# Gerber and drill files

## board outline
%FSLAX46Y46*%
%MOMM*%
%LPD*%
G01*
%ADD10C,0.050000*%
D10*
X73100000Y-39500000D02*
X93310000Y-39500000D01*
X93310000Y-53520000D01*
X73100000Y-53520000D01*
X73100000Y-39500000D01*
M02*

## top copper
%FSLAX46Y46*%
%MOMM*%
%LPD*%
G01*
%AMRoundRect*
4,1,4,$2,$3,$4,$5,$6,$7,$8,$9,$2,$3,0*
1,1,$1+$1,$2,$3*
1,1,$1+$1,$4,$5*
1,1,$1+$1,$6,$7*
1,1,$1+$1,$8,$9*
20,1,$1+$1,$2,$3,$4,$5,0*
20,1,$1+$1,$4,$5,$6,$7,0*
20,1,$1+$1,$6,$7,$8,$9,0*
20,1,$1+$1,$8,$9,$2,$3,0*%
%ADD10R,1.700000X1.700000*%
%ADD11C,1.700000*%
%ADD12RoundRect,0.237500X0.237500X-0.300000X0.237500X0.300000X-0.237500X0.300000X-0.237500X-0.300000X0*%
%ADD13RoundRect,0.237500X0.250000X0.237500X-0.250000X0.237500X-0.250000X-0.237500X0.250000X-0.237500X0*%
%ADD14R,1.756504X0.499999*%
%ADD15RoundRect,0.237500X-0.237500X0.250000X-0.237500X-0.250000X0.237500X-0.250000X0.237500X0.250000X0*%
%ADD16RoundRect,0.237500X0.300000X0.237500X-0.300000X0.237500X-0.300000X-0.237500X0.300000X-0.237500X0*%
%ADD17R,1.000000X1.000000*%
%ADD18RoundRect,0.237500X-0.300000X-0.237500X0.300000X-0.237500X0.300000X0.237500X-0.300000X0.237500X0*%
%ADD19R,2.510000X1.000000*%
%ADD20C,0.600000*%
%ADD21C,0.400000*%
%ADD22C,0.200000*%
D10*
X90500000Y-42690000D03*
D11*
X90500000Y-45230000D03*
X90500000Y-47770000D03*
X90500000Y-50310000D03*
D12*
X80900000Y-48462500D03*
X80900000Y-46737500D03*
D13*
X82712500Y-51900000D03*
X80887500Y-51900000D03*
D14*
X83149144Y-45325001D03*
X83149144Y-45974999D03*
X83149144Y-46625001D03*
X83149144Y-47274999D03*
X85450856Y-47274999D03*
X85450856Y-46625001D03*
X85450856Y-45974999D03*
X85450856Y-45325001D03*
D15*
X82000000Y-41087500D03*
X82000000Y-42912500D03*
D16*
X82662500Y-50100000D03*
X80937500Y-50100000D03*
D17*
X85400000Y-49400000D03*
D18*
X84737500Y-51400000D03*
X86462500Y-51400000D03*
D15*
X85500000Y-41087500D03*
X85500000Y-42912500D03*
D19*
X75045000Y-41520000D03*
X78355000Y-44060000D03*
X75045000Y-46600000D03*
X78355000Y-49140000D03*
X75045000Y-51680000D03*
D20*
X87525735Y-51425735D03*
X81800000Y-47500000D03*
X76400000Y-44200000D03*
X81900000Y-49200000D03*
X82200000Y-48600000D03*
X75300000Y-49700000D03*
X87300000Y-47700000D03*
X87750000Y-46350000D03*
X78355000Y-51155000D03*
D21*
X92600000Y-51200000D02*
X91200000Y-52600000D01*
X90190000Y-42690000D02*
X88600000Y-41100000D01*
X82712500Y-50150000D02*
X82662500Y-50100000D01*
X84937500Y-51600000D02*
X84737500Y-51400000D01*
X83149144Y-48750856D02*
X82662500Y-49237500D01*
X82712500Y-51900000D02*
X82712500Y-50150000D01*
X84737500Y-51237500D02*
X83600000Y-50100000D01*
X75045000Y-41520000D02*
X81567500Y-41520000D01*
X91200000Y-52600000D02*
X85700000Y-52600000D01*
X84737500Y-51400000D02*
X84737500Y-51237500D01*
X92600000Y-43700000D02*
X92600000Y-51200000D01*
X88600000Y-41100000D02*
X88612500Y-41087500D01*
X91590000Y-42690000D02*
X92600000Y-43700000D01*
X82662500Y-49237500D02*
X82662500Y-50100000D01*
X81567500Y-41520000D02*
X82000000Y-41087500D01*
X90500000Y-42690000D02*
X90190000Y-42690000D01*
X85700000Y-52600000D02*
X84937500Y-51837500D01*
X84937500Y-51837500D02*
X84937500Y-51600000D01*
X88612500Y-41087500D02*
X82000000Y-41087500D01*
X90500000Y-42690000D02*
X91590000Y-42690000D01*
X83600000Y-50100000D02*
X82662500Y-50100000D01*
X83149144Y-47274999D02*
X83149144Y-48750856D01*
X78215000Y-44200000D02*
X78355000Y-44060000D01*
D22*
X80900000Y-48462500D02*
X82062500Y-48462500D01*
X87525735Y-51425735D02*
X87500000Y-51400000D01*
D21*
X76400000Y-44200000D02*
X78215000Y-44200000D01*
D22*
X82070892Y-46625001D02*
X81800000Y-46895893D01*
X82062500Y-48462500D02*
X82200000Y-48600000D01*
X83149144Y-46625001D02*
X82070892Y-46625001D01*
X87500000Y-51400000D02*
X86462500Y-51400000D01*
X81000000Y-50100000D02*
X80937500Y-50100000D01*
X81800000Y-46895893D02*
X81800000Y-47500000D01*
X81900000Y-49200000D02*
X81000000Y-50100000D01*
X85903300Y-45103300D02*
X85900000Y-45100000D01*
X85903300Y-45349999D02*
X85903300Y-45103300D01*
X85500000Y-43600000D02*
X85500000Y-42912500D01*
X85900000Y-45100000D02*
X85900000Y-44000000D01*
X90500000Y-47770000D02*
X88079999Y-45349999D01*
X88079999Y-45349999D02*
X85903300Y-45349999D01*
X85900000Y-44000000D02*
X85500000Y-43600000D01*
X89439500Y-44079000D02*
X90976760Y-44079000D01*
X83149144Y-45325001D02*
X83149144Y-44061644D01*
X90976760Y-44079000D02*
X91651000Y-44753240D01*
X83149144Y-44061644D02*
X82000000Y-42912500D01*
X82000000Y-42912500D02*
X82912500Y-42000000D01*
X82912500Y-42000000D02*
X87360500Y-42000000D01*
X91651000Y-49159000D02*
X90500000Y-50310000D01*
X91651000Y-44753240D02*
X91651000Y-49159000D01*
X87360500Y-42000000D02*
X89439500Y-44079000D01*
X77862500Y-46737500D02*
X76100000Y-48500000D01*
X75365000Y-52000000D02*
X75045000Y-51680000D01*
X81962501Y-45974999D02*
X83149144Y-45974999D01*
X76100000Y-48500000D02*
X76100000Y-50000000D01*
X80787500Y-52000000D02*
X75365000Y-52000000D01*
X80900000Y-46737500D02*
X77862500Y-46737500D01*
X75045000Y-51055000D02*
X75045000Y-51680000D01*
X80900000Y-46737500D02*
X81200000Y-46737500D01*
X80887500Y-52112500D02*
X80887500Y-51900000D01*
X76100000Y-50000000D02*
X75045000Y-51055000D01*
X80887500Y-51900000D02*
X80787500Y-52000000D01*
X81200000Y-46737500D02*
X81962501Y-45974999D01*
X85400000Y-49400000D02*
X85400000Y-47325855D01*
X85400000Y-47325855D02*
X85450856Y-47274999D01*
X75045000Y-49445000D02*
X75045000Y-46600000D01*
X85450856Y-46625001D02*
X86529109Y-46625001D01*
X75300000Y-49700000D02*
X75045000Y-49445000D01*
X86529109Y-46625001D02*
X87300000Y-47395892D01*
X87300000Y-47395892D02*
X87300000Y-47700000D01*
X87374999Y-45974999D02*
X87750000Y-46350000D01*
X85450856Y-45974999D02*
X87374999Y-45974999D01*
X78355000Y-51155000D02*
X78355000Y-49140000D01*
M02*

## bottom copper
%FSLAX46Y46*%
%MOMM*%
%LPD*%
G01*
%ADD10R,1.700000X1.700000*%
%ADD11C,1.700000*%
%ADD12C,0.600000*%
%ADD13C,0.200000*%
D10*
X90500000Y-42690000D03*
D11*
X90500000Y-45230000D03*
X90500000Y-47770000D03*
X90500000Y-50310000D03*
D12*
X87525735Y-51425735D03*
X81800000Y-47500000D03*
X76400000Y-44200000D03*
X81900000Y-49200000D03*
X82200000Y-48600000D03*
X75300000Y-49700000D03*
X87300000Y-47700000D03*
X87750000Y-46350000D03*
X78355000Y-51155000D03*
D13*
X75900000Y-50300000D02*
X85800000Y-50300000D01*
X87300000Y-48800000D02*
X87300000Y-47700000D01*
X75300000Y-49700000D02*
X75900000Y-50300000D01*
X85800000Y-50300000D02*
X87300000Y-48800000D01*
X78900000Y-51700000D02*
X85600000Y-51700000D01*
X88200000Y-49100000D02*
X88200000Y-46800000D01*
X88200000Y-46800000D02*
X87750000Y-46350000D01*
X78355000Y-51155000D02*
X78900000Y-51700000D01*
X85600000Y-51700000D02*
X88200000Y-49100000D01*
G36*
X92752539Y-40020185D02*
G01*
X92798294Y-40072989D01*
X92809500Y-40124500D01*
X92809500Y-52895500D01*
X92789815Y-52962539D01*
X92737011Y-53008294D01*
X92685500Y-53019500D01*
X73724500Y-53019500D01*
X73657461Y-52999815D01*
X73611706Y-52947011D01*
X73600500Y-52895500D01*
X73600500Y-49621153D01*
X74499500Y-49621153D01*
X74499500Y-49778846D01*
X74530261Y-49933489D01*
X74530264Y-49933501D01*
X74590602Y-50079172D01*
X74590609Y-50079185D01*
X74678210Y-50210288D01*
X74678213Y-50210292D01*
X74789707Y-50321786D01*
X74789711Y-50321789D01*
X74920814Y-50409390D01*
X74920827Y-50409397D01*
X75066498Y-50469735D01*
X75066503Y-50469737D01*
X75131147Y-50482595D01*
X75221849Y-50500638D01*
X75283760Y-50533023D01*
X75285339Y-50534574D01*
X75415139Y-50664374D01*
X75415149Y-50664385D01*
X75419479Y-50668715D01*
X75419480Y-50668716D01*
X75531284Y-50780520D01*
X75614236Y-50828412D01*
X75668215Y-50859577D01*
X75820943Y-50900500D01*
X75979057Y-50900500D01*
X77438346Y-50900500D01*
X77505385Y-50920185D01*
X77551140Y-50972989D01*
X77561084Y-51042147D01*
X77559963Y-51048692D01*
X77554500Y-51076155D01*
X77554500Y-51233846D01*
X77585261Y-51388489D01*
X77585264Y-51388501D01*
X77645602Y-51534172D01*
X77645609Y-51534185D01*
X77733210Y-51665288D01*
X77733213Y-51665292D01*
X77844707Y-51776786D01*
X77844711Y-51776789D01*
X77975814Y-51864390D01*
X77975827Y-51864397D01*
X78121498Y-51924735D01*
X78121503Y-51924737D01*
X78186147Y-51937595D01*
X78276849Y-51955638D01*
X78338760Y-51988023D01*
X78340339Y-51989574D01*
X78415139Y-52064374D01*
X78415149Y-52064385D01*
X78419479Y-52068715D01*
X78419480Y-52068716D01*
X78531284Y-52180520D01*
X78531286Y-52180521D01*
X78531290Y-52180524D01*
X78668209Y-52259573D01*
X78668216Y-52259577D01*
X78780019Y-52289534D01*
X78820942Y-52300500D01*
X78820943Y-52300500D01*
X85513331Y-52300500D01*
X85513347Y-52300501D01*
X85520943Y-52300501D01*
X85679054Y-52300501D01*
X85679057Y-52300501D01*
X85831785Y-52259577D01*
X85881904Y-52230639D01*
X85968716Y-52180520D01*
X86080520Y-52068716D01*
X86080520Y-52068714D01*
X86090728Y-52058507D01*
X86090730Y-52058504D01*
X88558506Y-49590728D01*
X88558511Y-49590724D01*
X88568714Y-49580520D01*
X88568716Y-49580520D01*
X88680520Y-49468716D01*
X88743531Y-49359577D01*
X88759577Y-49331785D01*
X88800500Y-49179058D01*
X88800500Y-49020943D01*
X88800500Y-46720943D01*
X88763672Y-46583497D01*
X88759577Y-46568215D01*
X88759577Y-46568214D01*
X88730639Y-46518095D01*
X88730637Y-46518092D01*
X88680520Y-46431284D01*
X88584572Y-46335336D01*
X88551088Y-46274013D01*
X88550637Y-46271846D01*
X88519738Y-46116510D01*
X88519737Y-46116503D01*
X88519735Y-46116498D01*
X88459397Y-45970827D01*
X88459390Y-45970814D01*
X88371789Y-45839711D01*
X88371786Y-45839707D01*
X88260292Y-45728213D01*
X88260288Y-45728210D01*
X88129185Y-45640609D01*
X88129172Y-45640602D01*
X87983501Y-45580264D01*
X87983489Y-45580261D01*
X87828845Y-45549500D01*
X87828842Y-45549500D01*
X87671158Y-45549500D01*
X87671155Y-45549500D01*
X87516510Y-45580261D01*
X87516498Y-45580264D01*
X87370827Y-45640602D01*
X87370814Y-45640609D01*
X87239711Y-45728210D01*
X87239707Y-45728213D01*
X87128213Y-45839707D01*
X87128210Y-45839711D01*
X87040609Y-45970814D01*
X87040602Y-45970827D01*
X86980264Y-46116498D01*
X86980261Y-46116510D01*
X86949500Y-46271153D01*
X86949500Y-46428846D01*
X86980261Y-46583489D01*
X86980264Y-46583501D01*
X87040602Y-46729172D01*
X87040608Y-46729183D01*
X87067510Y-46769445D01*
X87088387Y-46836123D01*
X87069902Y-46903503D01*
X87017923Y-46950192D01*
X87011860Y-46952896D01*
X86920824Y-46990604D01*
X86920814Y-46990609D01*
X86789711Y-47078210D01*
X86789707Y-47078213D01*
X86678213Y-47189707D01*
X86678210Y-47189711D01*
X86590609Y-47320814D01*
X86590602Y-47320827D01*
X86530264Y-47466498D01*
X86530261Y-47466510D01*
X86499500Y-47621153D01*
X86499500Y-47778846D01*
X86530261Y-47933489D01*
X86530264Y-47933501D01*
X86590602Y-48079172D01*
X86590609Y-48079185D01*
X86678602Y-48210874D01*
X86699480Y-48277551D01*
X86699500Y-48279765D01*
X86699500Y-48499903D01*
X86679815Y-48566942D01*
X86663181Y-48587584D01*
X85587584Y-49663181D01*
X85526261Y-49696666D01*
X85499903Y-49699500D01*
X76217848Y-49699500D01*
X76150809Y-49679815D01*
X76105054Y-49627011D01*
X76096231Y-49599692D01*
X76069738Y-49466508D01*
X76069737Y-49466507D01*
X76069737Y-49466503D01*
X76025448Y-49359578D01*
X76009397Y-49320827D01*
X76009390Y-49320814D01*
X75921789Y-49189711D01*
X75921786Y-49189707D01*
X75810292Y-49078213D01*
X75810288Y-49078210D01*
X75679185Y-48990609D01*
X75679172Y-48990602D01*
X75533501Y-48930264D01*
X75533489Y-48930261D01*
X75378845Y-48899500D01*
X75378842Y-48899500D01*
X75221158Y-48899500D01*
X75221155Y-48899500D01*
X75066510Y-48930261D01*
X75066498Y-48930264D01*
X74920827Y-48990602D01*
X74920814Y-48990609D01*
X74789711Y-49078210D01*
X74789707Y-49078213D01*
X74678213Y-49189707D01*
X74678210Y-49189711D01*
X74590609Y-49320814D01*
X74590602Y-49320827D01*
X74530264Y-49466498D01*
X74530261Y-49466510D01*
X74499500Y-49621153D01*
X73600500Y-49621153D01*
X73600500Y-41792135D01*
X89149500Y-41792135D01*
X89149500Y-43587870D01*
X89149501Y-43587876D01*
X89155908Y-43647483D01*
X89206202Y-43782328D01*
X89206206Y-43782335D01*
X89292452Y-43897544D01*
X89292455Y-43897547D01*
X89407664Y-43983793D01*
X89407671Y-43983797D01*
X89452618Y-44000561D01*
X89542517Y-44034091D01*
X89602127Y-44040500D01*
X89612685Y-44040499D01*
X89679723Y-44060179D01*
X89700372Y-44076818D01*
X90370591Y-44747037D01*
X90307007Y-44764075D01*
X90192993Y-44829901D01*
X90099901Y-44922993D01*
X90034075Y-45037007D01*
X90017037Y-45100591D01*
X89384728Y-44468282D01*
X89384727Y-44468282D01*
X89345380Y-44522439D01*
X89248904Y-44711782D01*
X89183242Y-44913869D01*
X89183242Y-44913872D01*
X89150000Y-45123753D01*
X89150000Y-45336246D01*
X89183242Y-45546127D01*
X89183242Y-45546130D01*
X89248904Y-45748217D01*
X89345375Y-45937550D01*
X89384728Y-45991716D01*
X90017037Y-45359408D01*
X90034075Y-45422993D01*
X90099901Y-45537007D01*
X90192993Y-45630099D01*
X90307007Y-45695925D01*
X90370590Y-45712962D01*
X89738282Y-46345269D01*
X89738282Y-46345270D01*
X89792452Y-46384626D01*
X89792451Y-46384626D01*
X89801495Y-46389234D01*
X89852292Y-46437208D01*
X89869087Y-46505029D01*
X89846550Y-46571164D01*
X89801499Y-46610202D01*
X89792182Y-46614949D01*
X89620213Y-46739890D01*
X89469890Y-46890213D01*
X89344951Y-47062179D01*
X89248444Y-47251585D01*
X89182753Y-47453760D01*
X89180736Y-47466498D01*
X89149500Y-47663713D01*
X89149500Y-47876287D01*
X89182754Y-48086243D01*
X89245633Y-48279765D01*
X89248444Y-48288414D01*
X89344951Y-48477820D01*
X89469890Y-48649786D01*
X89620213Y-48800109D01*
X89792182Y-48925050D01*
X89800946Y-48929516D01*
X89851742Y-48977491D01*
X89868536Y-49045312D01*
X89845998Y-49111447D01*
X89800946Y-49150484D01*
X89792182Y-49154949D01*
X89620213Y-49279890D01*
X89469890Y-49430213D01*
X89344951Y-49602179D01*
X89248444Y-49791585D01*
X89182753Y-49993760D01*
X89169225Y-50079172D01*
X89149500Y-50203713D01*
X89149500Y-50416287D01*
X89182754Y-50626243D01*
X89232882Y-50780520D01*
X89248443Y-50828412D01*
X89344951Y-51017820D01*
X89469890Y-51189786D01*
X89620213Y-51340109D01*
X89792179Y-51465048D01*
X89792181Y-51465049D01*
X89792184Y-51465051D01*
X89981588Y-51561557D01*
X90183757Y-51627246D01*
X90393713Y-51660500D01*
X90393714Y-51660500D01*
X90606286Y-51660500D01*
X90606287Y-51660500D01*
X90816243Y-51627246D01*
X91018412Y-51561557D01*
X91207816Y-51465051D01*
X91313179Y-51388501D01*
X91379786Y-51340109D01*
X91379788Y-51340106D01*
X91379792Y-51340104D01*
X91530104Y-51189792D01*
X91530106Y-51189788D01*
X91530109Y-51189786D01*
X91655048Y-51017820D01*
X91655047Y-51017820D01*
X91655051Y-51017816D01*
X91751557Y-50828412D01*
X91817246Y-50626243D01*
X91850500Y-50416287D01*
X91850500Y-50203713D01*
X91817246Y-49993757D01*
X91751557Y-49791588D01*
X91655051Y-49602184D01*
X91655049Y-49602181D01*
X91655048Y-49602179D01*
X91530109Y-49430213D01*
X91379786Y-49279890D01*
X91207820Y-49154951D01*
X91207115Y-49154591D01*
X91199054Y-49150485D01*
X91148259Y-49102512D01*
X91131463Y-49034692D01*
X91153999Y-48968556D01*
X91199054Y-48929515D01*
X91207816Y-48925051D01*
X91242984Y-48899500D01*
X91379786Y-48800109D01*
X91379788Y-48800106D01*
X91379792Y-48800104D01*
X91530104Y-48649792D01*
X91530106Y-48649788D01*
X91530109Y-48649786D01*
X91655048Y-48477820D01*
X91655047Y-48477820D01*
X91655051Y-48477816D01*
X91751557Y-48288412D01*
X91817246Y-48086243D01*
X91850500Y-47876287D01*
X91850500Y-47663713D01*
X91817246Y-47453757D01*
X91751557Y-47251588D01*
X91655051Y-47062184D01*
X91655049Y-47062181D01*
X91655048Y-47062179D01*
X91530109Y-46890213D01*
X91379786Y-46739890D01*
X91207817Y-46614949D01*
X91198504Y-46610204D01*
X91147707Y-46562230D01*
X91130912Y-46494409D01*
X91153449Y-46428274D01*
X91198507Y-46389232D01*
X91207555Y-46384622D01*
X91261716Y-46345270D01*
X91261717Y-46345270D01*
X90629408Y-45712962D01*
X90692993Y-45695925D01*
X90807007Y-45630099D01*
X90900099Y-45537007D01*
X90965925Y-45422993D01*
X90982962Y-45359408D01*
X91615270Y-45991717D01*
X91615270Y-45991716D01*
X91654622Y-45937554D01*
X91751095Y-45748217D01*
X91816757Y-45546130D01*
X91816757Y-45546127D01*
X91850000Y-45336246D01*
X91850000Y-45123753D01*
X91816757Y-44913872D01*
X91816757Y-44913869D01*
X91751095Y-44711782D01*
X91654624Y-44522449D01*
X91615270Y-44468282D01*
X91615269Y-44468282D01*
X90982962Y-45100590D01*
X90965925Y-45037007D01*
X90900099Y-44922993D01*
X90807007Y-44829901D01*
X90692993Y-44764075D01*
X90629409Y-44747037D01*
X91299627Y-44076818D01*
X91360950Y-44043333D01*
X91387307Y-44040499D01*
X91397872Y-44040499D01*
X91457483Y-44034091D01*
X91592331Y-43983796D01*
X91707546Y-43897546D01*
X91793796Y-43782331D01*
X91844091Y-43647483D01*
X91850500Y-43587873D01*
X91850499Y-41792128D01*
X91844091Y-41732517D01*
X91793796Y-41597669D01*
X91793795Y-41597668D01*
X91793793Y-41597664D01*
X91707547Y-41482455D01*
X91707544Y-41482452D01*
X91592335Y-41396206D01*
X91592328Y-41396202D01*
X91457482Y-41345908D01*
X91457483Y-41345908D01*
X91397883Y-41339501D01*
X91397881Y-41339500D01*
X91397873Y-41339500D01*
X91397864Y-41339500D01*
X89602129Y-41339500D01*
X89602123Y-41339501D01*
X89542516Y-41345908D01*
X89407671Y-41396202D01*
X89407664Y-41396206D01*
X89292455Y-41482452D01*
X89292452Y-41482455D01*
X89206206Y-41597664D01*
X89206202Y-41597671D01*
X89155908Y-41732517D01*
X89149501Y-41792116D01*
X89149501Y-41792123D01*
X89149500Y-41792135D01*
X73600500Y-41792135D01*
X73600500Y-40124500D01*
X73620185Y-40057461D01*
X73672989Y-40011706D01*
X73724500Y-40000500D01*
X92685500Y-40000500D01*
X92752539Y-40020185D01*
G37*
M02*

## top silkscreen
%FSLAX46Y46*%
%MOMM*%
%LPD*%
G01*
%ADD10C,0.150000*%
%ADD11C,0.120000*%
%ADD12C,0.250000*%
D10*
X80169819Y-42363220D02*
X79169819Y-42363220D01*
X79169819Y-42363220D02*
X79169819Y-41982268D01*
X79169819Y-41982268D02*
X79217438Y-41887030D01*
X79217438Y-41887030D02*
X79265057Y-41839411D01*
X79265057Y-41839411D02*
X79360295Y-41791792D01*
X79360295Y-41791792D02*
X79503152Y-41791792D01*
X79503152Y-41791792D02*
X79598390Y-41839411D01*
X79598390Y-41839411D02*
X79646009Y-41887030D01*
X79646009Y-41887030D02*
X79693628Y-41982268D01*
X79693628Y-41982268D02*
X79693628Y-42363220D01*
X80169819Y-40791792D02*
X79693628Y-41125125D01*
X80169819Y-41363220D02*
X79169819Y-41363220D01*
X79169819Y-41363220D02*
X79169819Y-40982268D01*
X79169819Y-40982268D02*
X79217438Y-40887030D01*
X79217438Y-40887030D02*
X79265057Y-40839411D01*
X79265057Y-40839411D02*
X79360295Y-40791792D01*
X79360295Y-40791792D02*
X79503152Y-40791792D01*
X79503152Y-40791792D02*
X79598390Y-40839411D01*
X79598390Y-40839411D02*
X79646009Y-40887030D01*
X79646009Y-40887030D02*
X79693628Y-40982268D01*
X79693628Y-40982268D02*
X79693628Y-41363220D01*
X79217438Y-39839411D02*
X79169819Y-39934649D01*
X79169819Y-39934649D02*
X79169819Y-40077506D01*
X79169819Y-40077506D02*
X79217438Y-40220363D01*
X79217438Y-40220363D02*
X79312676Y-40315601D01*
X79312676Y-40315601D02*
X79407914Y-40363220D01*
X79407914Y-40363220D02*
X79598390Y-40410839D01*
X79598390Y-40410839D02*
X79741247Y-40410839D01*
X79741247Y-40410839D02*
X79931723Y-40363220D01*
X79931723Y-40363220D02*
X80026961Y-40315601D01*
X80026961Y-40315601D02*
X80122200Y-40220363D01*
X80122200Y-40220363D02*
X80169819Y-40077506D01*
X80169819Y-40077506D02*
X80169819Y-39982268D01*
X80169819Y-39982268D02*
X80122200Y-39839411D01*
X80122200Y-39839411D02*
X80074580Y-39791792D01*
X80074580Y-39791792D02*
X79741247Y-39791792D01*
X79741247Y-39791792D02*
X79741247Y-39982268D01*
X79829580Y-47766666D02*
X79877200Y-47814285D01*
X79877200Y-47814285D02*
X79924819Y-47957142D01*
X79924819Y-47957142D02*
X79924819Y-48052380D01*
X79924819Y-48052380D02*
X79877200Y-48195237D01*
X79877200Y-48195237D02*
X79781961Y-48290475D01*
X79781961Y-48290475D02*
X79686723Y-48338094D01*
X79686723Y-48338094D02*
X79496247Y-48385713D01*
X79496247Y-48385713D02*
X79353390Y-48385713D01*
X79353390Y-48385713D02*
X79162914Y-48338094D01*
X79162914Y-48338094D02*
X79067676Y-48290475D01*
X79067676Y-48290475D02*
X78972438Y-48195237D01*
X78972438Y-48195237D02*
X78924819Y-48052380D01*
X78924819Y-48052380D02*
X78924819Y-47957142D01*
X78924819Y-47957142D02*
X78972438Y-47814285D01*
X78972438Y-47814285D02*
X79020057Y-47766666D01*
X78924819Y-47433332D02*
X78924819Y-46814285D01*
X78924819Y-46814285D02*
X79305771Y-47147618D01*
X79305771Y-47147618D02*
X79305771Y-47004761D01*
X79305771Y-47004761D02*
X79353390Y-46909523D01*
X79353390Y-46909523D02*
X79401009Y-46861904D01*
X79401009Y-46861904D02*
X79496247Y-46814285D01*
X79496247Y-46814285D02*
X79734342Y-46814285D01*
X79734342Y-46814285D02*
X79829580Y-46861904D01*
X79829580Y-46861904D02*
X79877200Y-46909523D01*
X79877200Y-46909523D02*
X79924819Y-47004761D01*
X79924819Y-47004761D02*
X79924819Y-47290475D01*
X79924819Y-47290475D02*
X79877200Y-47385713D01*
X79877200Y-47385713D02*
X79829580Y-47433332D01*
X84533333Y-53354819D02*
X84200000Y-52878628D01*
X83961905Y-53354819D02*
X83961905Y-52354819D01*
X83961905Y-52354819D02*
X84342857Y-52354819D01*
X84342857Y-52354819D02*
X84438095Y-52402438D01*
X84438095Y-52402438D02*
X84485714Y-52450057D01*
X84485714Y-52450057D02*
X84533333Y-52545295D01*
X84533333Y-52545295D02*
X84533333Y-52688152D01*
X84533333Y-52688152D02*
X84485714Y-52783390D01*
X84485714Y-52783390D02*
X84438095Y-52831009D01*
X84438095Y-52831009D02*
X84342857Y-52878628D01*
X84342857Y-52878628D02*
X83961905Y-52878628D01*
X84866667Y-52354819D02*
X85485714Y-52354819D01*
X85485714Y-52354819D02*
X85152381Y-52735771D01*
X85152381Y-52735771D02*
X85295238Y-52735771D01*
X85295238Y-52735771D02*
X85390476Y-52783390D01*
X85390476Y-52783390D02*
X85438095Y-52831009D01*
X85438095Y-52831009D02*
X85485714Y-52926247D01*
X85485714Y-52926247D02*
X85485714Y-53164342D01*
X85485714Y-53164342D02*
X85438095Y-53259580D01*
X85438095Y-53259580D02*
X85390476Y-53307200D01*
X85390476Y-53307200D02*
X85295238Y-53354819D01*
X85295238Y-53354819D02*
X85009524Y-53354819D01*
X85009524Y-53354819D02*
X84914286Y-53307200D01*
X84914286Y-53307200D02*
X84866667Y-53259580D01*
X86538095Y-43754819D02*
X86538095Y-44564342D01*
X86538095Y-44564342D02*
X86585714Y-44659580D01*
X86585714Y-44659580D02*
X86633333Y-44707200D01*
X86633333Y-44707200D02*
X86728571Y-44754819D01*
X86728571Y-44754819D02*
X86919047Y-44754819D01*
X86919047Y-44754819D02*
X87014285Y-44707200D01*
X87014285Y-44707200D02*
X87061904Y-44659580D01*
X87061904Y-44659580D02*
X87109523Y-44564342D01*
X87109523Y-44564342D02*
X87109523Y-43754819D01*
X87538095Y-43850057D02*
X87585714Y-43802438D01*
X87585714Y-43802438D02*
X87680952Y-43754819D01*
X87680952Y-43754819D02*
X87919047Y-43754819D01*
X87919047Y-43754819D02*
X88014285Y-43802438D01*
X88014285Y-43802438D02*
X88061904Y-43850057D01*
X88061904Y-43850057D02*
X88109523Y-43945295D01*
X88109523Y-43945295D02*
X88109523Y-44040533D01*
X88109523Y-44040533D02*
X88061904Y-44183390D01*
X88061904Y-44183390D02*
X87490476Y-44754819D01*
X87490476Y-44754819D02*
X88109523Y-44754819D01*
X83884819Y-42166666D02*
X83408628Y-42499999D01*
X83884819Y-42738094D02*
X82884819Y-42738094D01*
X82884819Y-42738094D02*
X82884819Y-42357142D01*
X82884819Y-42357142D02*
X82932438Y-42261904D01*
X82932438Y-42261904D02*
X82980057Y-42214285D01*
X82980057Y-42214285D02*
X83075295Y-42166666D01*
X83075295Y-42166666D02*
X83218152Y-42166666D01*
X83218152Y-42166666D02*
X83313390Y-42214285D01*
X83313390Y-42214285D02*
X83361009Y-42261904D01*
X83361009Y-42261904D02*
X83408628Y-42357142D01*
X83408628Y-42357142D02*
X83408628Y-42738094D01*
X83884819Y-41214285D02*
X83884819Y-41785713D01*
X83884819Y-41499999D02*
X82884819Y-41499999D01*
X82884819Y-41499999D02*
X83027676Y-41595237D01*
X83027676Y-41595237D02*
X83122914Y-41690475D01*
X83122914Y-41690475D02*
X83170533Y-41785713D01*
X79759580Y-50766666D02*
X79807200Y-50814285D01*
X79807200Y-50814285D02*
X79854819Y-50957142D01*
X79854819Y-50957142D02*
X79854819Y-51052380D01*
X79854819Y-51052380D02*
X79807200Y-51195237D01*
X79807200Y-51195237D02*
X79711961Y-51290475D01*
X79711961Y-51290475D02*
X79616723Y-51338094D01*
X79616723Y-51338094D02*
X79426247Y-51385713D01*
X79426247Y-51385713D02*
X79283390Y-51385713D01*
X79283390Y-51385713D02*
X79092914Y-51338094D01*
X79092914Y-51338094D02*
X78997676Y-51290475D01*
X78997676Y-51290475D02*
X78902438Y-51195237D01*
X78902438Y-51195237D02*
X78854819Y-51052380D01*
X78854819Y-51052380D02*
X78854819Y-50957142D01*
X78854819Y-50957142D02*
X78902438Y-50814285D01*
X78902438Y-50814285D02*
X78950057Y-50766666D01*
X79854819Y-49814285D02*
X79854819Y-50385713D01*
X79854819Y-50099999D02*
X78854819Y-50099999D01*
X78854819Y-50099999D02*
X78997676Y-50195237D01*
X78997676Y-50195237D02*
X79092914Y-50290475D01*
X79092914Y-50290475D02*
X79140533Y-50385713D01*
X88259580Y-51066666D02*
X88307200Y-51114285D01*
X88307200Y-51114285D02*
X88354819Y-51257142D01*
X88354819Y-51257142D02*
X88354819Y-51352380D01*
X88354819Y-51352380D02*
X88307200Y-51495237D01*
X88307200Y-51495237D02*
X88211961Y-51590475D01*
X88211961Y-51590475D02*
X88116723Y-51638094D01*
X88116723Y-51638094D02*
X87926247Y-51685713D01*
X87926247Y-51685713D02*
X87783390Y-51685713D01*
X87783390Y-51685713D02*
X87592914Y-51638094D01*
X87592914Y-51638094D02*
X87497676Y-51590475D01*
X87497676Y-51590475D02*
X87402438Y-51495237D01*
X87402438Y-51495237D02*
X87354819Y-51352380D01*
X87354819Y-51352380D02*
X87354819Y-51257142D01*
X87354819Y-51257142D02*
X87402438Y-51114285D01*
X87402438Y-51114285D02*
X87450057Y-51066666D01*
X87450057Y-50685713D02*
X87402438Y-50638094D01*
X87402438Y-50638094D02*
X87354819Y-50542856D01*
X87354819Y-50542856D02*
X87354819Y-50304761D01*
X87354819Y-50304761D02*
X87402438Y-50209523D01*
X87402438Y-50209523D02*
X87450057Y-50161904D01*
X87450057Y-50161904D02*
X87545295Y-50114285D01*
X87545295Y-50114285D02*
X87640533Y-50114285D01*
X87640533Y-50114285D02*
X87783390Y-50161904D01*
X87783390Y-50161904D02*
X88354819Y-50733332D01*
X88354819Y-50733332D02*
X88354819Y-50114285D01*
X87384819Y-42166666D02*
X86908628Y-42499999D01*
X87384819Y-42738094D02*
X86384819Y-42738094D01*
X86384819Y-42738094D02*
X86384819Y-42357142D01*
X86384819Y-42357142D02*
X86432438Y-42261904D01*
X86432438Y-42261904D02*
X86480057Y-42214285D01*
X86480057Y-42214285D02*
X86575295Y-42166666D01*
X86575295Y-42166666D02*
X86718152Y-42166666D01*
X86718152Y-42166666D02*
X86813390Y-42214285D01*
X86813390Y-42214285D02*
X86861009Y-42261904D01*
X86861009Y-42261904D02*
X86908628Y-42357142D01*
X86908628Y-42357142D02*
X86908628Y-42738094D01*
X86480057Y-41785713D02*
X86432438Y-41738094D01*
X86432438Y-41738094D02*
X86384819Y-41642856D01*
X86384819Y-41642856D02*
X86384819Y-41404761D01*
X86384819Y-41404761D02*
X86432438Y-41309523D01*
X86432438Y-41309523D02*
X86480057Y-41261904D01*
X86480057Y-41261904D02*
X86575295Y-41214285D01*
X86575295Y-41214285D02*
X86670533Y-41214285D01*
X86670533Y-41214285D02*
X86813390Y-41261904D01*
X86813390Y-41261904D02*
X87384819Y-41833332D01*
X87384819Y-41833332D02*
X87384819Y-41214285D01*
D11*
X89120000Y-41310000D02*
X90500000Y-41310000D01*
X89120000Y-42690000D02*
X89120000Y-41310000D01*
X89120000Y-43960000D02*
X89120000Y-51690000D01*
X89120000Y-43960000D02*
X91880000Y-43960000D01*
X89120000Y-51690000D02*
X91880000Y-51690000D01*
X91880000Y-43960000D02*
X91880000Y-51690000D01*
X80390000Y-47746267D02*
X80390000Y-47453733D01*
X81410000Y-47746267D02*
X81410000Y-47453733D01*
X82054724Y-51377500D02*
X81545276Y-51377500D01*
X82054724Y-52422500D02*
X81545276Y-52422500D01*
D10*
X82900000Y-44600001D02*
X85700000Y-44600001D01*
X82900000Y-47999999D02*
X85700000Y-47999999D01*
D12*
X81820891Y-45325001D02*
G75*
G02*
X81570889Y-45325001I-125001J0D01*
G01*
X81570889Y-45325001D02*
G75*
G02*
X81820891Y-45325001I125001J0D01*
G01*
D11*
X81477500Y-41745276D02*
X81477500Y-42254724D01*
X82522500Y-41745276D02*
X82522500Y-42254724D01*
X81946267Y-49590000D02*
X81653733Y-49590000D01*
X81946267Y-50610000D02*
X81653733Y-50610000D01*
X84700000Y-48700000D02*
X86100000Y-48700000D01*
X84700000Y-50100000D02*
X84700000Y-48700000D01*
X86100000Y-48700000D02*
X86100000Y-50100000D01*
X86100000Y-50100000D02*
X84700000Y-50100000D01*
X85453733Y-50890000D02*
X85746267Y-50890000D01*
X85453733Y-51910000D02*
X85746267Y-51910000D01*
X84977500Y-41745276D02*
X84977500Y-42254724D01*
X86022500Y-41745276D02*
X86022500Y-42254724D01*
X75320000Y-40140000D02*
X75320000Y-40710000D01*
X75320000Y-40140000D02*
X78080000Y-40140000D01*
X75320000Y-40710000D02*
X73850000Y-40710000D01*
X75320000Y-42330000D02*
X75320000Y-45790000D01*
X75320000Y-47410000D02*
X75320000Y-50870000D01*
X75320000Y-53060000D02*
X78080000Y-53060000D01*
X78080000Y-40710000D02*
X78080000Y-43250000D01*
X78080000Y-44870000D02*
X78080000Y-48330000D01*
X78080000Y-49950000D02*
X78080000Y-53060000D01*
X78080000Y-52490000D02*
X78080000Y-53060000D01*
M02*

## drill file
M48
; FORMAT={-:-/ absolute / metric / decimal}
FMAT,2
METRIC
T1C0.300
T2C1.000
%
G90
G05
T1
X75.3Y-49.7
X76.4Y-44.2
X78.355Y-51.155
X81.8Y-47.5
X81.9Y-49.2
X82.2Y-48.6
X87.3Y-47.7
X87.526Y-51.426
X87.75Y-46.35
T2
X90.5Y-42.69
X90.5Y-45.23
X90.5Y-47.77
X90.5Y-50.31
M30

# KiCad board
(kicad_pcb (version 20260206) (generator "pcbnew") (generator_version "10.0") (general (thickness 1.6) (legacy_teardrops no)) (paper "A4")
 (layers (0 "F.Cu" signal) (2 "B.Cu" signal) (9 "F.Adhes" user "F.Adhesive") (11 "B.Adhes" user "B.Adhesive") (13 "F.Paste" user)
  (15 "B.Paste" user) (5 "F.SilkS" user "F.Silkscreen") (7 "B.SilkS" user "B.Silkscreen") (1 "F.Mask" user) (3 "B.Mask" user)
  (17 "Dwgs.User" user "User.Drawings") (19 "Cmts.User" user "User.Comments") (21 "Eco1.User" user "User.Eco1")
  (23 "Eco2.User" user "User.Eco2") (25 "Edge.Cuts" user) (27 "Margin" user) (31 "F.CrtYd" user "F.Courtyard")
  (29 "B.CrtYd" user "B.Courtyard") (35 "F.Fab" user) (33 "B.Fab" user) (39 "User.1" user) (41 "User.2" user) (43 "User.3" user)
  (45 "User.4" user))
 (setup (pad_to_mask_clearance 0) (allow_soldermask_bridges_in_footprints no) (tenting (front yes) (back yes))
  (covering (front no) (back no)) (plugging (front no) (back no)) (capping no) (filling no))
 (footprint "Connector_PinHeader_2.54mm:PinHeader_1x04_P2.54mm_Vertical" (layer "F.Cu") (at 90.5 42.69)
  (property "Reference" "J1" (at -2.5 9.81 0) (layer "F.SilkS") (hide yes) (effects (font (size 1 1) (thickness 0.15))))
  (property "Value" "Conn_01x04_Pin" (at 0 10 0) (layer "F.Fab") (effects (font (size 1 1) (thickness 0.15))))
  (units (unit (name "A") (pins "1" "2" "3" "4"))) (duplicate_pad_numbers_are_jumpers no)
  (fp_line (start -1.38 -1.38) (end 0 -1.38) (stroke (width 0.12) (type solid)) (layer "F.SilkS"))
  (fp_line (start -1.38 0) (end -1.38 -1.38) (stroke (width 0.12) (type solid)) (layer "F.SilkS"))
  (fp_line (start -1.38 1.27) (end -1.38 9) (stroke (width 0.12) (type solid)) (layer "F.SilkS"))
  (fp_line (start -1.38 1.27) (end 1.38 1.27) (stroke (width 0.12) (type solid)) (layer "F.SilkS"))
  (fp_line (start -1.38 9) (end 1.38 9) (stroke (width 0.12) (type solid)) (layer "F.SilkS"))
  (fp_line (start 1.38 1.27) (end 1.38 9) (stroke (width 0.12) (type solid)) (layer "F.SilkS"))
  (pad "1" thru_hole rect (at 0 0) (size 1.7 1.7) (drill 1) (layers "*.Cu" "*.Mask") (remove_unused_layers no) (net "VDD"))
  (pad "2" thru_hole circle (at 0 2.54) (size 1.7 1.7) (drill 1) (layers "*.Cu" "*.Mask") (remove_unused_layers no) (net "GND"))
  (pad "3" thru_hole circle (at 0 5.08) (size 1.7 1.7) (drill 1) (layers "*.Cu" "*.Mask") (remove_unused_layers no) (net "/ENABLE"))
  (pad "4" thru_hole circle (at 0 7.62) (size 1.7 1.7) (drill 1) (layers "*.Cu" "*.Mask") (remove_unused_layers no) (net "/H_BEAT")))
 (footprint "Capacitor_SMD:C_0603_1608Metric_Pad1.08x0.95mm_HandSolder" (layer "F.Cu") (at 80.9 47.6 90)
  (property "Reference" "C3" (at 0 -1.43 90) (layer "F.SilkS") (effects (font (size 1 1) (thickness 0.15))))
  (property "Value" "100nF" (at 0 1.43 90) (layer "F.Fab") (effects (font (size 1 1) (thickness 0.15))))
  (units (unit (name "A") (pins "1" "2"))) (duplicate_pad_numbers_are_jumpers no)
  (fp_line (start -0.146267 -0.51) (end 0.146267 -0.51) (stroke (width 0.12) (type solid)) (layer "F.SilkS"))
  (fp_line (start -0.146267 0.51) (end 0.146267 0.51) (stroke (width 0.12) (type solid)) (layer "F.SilkS"))
  (pad "1" smd roundrect (at -0.8625 0 90) (size 1.075 0.95) (layers "F.Cu" "F.Mask" "F.Paste") (roundrect_rratio 0.25) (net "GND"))
  (pad "2" smd roundrect (at 0.8625 0 90) (size 1.075 0.95) (layers "F.Cu" "F.Mask" "F.Paste") (roundrect_rratio 0.25) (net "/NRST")))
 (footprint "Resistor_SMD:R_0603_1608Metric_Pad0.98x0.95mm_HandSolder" (layer "F.Cu") (at 81.8 51.9 180)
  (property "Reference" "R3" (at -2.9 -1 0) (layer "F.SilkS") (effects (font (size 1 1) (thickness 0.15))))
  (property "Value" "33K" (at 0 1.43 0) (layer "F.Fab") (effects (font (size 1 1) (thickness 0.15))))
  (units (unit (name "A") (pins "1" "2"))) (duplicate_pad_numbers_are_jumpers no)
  (fp_line (start -0.254724 0.5225) (end 0.254724 0.5225) (stroke (width 0.12) (type solid)) (layer "F.SilkS"))
  (fp_line (start -0.254724 -0.5225) (end 0.254724 -0.5225) (stroke (width 0.12) (type solid)) (layer "F.SilkS"))
  (pad "1" smd roundrect (at -0.9125 0 180) (size 0.975 0.95) (layers "F.Cu" "F.Mask" "F.Paste") (roundrect_rratio 0.25) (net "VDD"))
  (pad "2" smd roundrect (at 0.9125 0 180) (size 0.975 0.95) (layers "F.Cu" "F.Mask" "F.Paste") (roundrect_rratio 0.25) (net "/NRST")))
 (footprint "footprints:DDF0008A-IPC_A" (layer "F.Cu") (at 84.3 46.3)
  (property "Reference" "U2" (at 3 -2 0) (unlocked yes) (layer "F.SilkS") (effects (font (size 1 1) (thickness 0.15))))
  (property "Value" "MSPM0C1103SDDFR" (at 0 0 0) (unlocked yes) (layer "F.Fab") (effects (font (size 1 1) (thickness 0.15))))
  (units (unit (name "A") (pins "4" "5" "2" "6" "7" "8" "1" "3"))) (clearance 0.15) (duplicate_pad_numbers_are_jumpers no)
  (fp_line (start -1.4 -1.699999) (end 1.4 -1.699999) (stroke (width 0.15) (type solid)) (layer "F.SilkS"))
  (fp_line (start -1.4 1.699999) (end 1.4 1.699999) (stroke (width 0.15) (type solid)) (layer "F.SilkS"))
  (fp_circle (center -2.60411 -0.974999) (end -2.479109 -0.974999) (stroke (width 0.25) (type solid)) (fill no) (layer "F.SilkS"))
  (pad "1" smd rect (at -1.150856 -0.974999) (size 1.756504 0.499999) (layers "F.Cu" "F.Mask" "F.Paste") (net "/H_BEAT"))
  (pad "2" smd rect (at -1.150856 -0.325001) (size 1.756504 0.499999) (layers "F.Cu" "F.Mask" "F.Paste") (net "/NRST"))
  (pad "3" smd rect (at -1.150856 0.325001) (size 1.756504 0.499999) (layers "F.Cu" "F.Mask" "F.Paste") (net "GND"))
  (pad "4" smd rect (at -1.150856 0.974999) (size 1.756504 0.499999) (layers "F.Cu" "F.Mask" "F.Paste") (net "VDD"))
  (pad "5" smd rect (at 1.150856 0.974999) (size 1.756504 0.499999) (layers "F.Cu" "F.Mask" "F.Paste") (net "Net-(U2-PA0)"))
  (pad "6" smd rect (at 1.150856 0.325001) (size 1.756504 0.499999) (layers "F.Cu" "F.Mask" "F.Paste") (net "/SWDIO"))
  (pad "7" smd rect (at 1.150856 -0.325001) (size 1.756504 0.499999) (layers "F.Cu" "F.Mask" "F.Paste") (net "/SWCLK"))
  (pad "8" smd rect (at 1.150856 -0.974999) (size 1.756504 0.499999) (layers "F.Cu" "F.Mask" "F.Paste") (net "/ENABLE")))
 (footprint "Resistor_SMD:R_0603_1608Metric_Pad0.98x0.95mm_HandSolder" (layer "F.Cu") (at 82 42 -90)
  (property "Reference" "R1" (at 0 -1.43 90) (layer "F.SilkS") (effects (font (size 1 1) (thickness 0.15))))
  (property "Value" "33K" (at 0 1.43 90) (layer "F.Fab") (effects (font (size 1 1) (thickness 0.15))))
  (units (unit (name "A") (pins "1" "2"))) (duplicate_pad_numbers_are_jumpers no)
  (fp_line (start -0.254724 0.5225) (end 0.254724 0.5225) (stroke (width 0.12) (type solid)) (layer "F.SilkS"))
  (fp_line (start -0.254724 -0.5225) (end 0.254724 -0.5225) (stroke (width 0.12) (type solid)) (layer "F.SilkS"))
  (pad "1" smd roundrect (at -0.9125 0 270) (size 0.975 0.95) (layers "F.Cu" "F.Mask" "F.Paste") (roundrect_rratio 0.25) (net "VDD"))
  (pad "2" smd roundrect (at 0.9125 0 270) (size 0.975 0.95) (layers "F.Cu" "F.Mask" "F.Paste") (roundrect_rratio 0.25) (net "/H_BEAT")))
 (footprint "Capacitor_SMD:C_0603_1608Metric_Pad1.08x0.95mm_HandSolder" (layer "F.Cu") (at 81.8 50.1 180)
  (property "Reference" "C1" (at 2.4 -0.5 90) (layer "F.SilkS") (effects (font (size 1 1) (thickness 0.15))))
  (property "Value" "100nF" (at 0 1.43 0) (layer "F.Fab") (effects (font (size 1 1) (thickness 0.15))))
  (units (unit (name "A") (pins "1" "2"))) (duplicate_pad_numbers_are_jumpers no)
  (fp_line (start -0.146267 0.51) (end 0.146267 0.51) (stroke (width 0.12) (type solid)) (layer "F.SilkS"))
  (fp_line (start -0.146267 -0.51) (end 0.146267 -0.51) (stroke (width 0.12) (type solid)) (layer "F.SilkS"))
  (pad "1" smd roundrect (at -0.8625 0 180) (size 1.075 0.95) (layers "F.Cu" "F.Mask" "F.Paste") (roundrect_rratio 0.25) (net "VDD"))
  (pad "2" smd roundrect (at 0.8625 0 180) (size 1.075 0.95) (layers "F.Cu" "F.Mask" "F.Paste") (roundrect_rratio 0.25) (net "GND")))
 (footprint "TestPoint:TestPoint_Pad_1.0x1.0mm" (layer "F.Cu") (at 85.4 49.4)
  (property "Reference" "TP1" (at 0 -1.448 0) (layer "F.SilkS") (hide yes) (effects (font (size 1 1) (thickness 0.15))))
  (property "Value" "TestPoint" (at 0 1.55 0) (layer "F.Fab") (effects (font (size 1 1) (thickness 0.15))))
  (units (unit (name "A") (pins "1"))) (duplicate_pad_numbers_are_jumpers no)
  (fp_line (start -0.7 -0.7) (end 0.7 -0.7) (stroke (width 0.12) (type solid)) (layer "F.SilkS"))
  (fp_line (start -0.7 0.7) (end -0.7 -0.7) (stroke (width 0.12) (type solid)) (layer "F.SilkS"))
  (fp_line (start 0.7 -0.7) (end 0.7 0.7) (stroke (width 0.12) (type solid)) (layer "F.SilkS"))
  (fp_line (start 0.7 0.7) (end -0.7 0.7) (stroke (width 0.12) (type solid)) (layer "F.SilkS"))
  (pad "1" smd rect (at 0 0) (size 1 1) (layers "F.Cu" "F.Mask") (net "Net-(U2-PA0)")))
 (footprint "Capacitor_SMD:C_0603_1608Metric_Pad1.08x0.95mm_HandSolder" (layer "F.Cu") (at 85.6 51.4)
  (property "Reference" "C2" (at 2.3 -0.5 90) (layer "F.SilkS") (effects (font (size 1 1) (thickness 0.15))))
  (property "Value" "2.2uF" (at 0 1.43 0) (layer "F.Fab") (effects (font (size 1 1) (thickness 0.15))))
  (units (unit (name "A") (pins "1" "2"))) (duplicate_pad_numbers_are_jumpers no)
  (fp_line (start -0.146267 -0.51) (end 0.146267 -0.51) (stroke (width 0.12) (type solid)) (layer "F.SilkS"))
  (fp_line (start -0.146267 0.51) (end 0.146267 0.51) (stroke (width 0.12) (type solid)) (layer "F.SilkS"))
  (pad "1" smd roundrect (at -0.8625 0) (size 1.075 0.95) (layers "F.Cu" "F.Mask" "F.Paste") (roundrect_rratio 0.25) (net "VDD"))
  (pad "2" smd roundrect (at 0.8625 0) (size 1.075 0.95) (layers "F.Cu" "F.Mask" "F.Paste") (roundrect_rratio 0.25) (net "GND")))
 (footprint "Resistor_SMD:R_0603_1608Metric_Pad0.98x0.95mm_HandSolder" (layer "F.Cu") (at 85.5 42 -90)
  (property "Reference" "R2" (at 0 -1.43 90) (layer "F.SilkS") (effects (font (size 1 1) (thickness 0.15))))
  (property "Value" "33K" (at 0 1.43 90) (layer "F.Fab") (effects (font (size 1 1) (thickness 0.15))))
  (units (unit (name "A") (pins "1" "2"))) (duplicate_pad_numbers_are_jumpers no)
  (fp_line (start -0.254724 0.5225) (end 0.254724 0.5225) (stroke (width 0.12) (type solid)) (layer "F.SilkS"))
  (fp_line (start -0.254724 -0.5225) (end 0.254724 -0.5225) (stroke (width 0.12) (type solid)) (layer "F.SilkS"))
  (pad "1" smd roundrect (at -0.9125 0 270) (size 0.975 0.95) (layers "F.Cu" "F.Mask" "F.Paste") (roundrect_rratio 0.25) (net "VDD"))
  (pad "2" smd roundrect (at 0.9125 0 270) (size 0.975 0.95) (layers "F.Cu" "F.Mask" "F.Paste") (roundrect_rratio 0.25) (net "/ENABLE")))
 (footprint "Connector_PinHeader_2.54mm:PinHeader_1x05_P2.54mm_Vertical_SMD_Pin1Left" (layer "F.Cu") (at 76.7 46.6)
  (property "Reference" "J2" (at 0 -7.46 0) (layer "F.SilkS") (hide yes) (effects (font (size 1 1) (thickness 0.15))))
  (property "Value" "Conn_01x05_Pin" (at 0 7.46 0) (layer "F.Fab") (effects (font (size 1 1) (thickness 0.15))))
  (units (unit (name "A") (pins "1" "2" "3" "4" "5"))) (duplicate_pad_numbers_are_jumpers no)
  (fp_line (start -1.38 -6.46) (end -1.38 -5.89) (stroke (width 0.12) (type solid)) (layer "F.SilkS"))
  (fp_line (start -1.38 -6.46) (end 1.38 -6.46) (stroke (width 0.12) (type solid)) (layer "F.SilkS"))
  (fp_line (start -1.38 -5.89) (end -2.85 -5.89) (stroke (width 0.12) (type solid)) (layer "F.SilkS"))
  (fp_line (start -1.38 -4.27) (end -1.38 -0.81) (stroke (width 0.12) (type solid)) (layer "F.SilkS"))
  (fp_line (start -1.38 0.81) (end -1.38 4.27) (stroke (width 0.12) (type solid)) (layer "F.SilkS"))
  (fp_line (start -1.38 6.46) (end 1.38 6.46) (stroke (width 0.12) (type solid)) (layer "F.SilkS"))
  (fp_line (start 1.38 -5.89) (end 1.38 -3.35) (stroke (width 0.12) (type solid)) (layer "F.SilkS"))
  (fp_line (start 1.38 -1.73) (end 1.38 1.73) (stroke (width 0.12) (type solid)) (layer "F.SilkS"))
  (fp_line (start 1.38 3.35) (end 1.38 6.46) (stroke (width 0.12) (type solid)) (layer "F.SilkS"))
  (fp_line (start 1.38 5.89) (end 1.38 6.46) (stroke (width 0.12) (type solid)) (layer "F.SilkS"))
  (pad "1" smd rect (at -1.655 -5.08) (size 2.51 1) (layers "F.Cu" "F.Mask" "F.Paste") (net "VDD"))
  (pad "2" smd rect (at 1.655 -2.54) (size 2.51 1) (layers "F.Cu" "F.Mask" "F.Paste") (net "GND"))
  (pad "3" smd rect (at -1.655 0) (size 2.51 1) (layers "F.Cu" "F.Mask" "F.Paste") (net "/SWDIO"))
  (pad "4" smd rect (at 1.655 2.54) (size 2.51 1) (layers "F.Cu" "F.Mask" "F.Paste") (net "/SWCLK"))
  (pad "5" smd rect (at -1.655 5.08) (size 2.51 1) (layers "F.Cu" "F.Mask" "F.Paste") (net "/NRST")))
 (gr_rect (start 73.1 39.5) (end 93.31 53.52) (stroke (width 0.05) (type default)) (fill no) (layer "Edge.Cuts"))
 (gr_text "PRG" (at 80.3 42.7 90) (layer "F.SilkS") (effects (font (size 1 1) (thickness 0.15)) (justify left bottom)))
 (segment (start 92.6 51.2) (end 91.2 52.6) (width 0.4) (layer "F.Cu") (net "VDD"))
 (segment (start 90.19 42.69) (end 88.6 41.1) (width 0.4) (layer "F.Cu") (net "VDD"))
 (segment (start 82.7125 50.15) (end 82.6625 50.1) (width 0.4) (layer "F.Cu") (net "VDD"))
 (segment (start 84.9375 51.6) (end 84.7375 51.4) (width 0.4) (layer "F.Cu") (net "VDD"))
 (segment (start 83.149144 48.750856) (end 82.6625 49.2375) (width 0.4) (layer "F.Cu") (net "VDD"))
 (segment (start 82.7125 51.9) (end 82.7125 50.15) (width 0.4) (layer "F.Cu") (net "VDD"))
 (segment (start 84.7375 51.2375) (end 83.6 50.1) (width 0.4) (layer "F.Cu") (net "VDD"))
 (segment (start 75.045 41.52) (end 81.5675 41.52) (width 0.4) (layer "F.Cu") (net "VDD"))
 (segment (start 91.2 52.6) (end 85.7 52.6) (width 0.4) (layer "F.Cu") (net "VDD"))
 (segment (start 84.7375 51.4) (end 84.7375 51.2375) (width 0.4) (layer "F.Cu") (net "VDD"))
 (segment (start 92.6 43.7) (end 92.6 51.2) (width 0.4) (layer "F.Cu") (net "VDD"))
 (segment (start 88.6 41.1) (end 88.6125 41.0875) (width 0.4) (layer "F.Cu") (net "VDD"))
 (segment (start 91.59 42.69) (end 92.6 43.7) (width 0.4) (layer "F.Cu") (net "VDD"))
 (segment (start 82.6625 49.2375) (end 82.6625 50.1) (width 0.4) (layer "F.Cu") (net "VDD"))
 (segment (start 81.5675 41.52) (end 82 41.0875) (width 0.4) (layer "F.Cu") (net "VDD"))
 (segment (start 90.5 42.69) (end 90.19 42.69) (width 0.4) (layer "F.Cu") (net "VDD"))
 (segment (start 85.7 52.6) (end 84.9375 51.8375) (width 0.4) (layer "F.Cu") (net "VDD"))
 (segment (start 84.9375 51.8375) (end 84.9375 51.6) (width 0.4) (layer "F.Cu") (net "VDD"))
 (segment (start 88.6125 41.0875) (end 82 41.0875) (width 0.4) (layer "F.Cu") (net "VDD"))
 (segment (start 90.5 42.69) (end 91.59 42.69) (width 0.4) (layer "F.Cu") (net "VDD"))
 (segment (start 83.6 50.1) (end 82.6625 50.1) (width 0.4) (layer "F.Cu") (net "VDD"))
 (segment (start 83.149144 47.274999) (end 83.149144 48.750856) (width 0.4) (layer "F.Cu") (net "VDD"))
 (segment (start 78.215 44.2) (end 78.355 44.06) (width 0.4) (layer "F.Cu") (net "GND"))
 (segment (start 80.9 48.4625) (end 82.0625 48.4625) (width 0.2) (layer "F.Cu") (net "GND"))
 (segment (start 87.525735 51.425735) (end 87.5 51.4) (width 0.2) (layer "F.Cu") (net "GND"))
 (segment (start 76.4 44.2) (end 78.215 44.2) (width 0.4) (layer "F.Cu") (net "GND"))
 (segment (start 82.070892 46.625001) (end 81.8 46.895893) (width 0.2) (layer "F.Cu") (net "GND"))
 (segment (start 82.0625 48.4625) (end 82.2 48.6) (width 0.2) (layer "F.Cu") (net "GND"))
 (segment (start 83.149144 46.625001) (end 82.070892 46.625001) (width 0.2) (layer "F.Cu") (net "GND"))
 (segment (start 87.5 51.4) (end 86.4625 51.4) (width 0.2) (layer "F.Cu") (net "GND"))
 (segment (start 81 50.1) (end 80.9375 50.1) (width 0.2) (layer "F.Cu") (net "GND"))
 (segment (start 81.8 46.895893) (end 81.8 47.5) (width 0.2) (layer "F.Cu") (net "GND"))
 (segment (start 81.9 49.2) (end 81 50.1) (width 0.2) (layer "F.Cu") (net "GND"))
 (via (at 87.525735 51.425735) (size 0.6) (drill 0.3) (layers "F.Cu" "B.Cu") (capping no) (covering (front no) (back no))
  (plugging (front no) (back no)) (filling no) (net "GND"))
 (via (at 81.8 47.5) (size 0.6) (drill 0.3) (layers "F.Cu" "B.Cu") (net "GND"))
 (via (at 76.4 44.2) (size 0.6) (drill 0.3) (layers "F.Cu" "B.Cu") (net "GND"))
 (via (at 81.9 49.2) (size 0.6) (drill 0.3) (layers "F.Cu" "B.Cu") (capping no) (covering (front no) (back no))
  (plugging (front no) (back no)) (filling no) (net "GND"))
 (via (at 82.2 48.6) (size 0.6) (drill 0.3) (layers "F.Cu" "B.Cu") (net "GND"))
 (segment (start 85.9033 45.1033) (end 85.9 45.1) (width 0.2) (layer "F.Cu") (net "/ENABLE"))
 (segment (start 85.9033 45.349999) (end 85.9033 45.1033) (width 0.2) (layer "F.Cu") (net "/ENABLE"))
 (segment (start 85.5 43.6) (end 85.5 42.9125) (width 0.2) (layer "F.Cu") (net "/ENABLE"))
 (segment (start 85.9 45.1) (end 85.9 44) (width 0.2) (layer "F.Cu") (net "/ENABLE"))
 (segment (start 90.5 47.77) (end 88.079999 45.349999) (width 0.2) (layer "F.Cu") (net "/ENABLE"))
 (segment (start 88.079999 45.349999) (end 85.9033 45.349999) (width 0.2) (layer "F.Cu") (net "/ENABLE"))
 (segment (start 85.9 44) (end 85.5 43.6) (width 0.2) (layer "F.Cu") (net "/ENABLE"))
 (segment (start 89.4395 44.079) (end 90.97676 44.079) (width 0.2) (layer "F.Cu") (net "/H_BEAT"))
 (segment (start 83.149144 45.325001) (end 83.149144 44.061644) (width 0.2) (layer "F.Cu") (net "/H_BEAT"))
 (segment (start 90.97676 44.079) (end 91.651 44.75324) (width 0.2) (layer "F.Cu") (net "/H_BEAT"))
 (segment (start 83.149144 44.061644) (end 82 42.9125) (width 0.2) (layer "F.Cu") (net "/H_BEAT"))
 (segment (start 82 42.9125) (end 82.9125 42) (width 0.2) (layer "F.Cu") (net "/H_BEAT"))
 (segment (start 82.9125 42) (end 87.3605 42) (width 0.2) (layer "F.Cu") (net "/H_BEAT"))
 (segment (start 91.651 49.159) (end 90.5 50.31) (width 0.2) (layer "F.Cu") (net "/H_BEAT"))
 (segment (start 91.651 44.75324) (end 91.651 49.159) (width 0.2) (layer "F.Cu") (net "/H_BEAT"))
 (segment (start 87.3605 42) (end 89.4395 44.079) (width 0.2) (layer "F.Cu") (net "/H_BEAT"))
 (segment (start 77.8625 46.7375) (end 76.1 48.5) (width 0.2) (layer "F.Cu") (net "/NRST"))
 (segment (start 75.365 52) (end 75.045 51.68) (width 0.2) (layer "F.Cu") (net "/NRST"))
 (segment (start 81.962501 45.974999) (end 83.149144 45.974999) (width 0.2) (layer "F.Cu") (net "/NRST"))
 (segment (start 76.1 48.5) (end 76.1 50) (width 0.2) (layer "F.Cu") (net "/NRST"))
 (segment (start 80.7875 52) (end 75.365 52) (width 0.2) (layer "F.Cu") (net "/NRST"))
 (segment (start 80.9 46.7375) (end 77.8625 46.7375) (width 0.2) (layer "F.Cu") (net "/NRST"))
 (segment (start 75.045 51.055) (end 75.045 51.68) (width 0.2) (layer "F.Cu") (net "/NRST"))
 (segment (start 80.9 46.7375) (end 81.2 46.7375) (width 0.2) (layer "F.Cu") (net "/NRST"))
 (segment (start 80.8875 52.1125) (end 80.8875 51.9) (width 0.2) (layer "F.Cu") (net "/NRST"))
 (segment (start 76.1 50) (end 75.045 51.055) (width 0.2) (layer "F.Cu") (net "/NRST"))
 (segment (start 80.8875 51.9) (end 80.7875 52) (width 0.2) (layer "F.Cu") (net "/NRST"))
 (segment (start 81.2 46.7375) (end 81.962501 45.974999) (width 0.2) (layer "F.Cu") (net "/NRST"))
 (segment (start 85.4 49.4) (end 85.4 47.325855) (width 0.2) (layer "F.Cu") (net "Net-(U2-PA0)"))
 (segment (start 85.4 47.325855) (end 85.450856 47.274999) (width 0.2) (layer "F.Cu") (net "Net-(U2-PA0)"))
 (segment (start 75.045 49.445) (end 75.045 46.6) (width 0.2) (layer "F.Cu") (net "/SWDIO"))
 (segment (start 85.450856 46.625001) (end 86.529109 46.625001) (width 0.2) (layer "F.Cu") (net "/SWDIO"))
 (segment (start 75.3 49.7) (end 75.045 49.445) (width 0.2) (layer "F.Cu") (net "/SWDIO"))
 (segment (start 86.529109 46.625001) (end 87.3 47.395892) (width 0.2) (layer "F.Cu") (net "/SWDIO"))
 (segment (start 87.3 47.395892) (end 87.3 47.7) (width 0.2) (layer "F.Cu") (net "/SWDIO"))
 (via (at 75.3 49.7) (size 0.6) (drill 0.3) (layers "F.Cu" "B.Cu") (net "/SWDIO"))
 (via (at 87.3 47.7) (size 0.6) (drill 0.3) (layers "F.Cu" "B.Cu") (capping no) (covering (front no) (back no))
  (plugging (front no) (back no)) (filling no) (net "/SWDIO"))
 (segment (start 75.9 50.3) (end 85.8 50.3) (width 0.2) (layer "B.Cu") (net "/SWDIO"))
 (segment (start 87.3 48.8) (end 87.3 47.7) (width 0.2) (layer "B.Cu") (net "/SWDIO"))
 (segment (start 75.3 49.7) (end 75.9 50.3) (width 0.2) (layer "B.Cu") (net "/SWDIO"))
 (segment (start 85.8 50.3) (end 87.3 48.8) (width 0.2) (layer "B.Cu") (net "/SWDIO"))
 (segment (start 87.374999 45.974999) (end 87.75 46.35) (width 0.2) (layer "F.Cu") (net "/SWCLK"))
 (segment (start 85.450856 45.974999) (end 87.374999 45.974999) (width 0.2) (layer "F.Cu") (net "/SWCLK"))
 (segment (start 78.355 51.155) (end 78.355 49.14) (width 0.2) (layer "F.Cu") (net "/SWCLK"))
 (via (at 87.75 46.35) (size 0.6) (drill 0.3) (layers "F.Cu" "B.Cu") (capping no) (covering (front no) (back no))
  (plugging (front no) (back no)) (filling no) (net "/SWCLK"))
 (via (at 78.355 51.155) (size 0.6) (drill 0.3) (layers "F.Cu" "B.Cu") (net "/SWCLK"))
 (segment (start 78.9 51.7) (end 85.6 51.7) (width 0.2) (layer "B.Cu") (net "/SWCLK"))
 (segment (start 88.2 49.1) (end 88.2 46.8) (width 0.2) (layer "B.Cu") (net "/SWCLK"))
 (segment (start 88.2 46.8) (end 87.75 46.35) (width 0.2) (layer "B.Cu") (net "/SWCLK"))
 (segment (start 78.355 51.155) (end 78.9 51.7) (width 0.2) (layer "B.Cu") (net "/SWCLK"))
 (segment (start 85.6 51.7) (end 88.2 49.1) (width 0.2) (layer "B.Cu") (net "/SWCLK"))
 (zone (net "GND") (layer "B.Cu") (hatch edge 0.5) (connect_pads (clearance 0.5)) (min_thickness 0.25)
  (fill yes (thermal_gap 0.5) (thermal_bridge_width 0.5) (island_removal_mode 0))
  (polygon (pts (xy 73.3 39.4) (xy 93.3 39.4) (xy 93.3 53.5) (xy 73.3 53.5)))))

